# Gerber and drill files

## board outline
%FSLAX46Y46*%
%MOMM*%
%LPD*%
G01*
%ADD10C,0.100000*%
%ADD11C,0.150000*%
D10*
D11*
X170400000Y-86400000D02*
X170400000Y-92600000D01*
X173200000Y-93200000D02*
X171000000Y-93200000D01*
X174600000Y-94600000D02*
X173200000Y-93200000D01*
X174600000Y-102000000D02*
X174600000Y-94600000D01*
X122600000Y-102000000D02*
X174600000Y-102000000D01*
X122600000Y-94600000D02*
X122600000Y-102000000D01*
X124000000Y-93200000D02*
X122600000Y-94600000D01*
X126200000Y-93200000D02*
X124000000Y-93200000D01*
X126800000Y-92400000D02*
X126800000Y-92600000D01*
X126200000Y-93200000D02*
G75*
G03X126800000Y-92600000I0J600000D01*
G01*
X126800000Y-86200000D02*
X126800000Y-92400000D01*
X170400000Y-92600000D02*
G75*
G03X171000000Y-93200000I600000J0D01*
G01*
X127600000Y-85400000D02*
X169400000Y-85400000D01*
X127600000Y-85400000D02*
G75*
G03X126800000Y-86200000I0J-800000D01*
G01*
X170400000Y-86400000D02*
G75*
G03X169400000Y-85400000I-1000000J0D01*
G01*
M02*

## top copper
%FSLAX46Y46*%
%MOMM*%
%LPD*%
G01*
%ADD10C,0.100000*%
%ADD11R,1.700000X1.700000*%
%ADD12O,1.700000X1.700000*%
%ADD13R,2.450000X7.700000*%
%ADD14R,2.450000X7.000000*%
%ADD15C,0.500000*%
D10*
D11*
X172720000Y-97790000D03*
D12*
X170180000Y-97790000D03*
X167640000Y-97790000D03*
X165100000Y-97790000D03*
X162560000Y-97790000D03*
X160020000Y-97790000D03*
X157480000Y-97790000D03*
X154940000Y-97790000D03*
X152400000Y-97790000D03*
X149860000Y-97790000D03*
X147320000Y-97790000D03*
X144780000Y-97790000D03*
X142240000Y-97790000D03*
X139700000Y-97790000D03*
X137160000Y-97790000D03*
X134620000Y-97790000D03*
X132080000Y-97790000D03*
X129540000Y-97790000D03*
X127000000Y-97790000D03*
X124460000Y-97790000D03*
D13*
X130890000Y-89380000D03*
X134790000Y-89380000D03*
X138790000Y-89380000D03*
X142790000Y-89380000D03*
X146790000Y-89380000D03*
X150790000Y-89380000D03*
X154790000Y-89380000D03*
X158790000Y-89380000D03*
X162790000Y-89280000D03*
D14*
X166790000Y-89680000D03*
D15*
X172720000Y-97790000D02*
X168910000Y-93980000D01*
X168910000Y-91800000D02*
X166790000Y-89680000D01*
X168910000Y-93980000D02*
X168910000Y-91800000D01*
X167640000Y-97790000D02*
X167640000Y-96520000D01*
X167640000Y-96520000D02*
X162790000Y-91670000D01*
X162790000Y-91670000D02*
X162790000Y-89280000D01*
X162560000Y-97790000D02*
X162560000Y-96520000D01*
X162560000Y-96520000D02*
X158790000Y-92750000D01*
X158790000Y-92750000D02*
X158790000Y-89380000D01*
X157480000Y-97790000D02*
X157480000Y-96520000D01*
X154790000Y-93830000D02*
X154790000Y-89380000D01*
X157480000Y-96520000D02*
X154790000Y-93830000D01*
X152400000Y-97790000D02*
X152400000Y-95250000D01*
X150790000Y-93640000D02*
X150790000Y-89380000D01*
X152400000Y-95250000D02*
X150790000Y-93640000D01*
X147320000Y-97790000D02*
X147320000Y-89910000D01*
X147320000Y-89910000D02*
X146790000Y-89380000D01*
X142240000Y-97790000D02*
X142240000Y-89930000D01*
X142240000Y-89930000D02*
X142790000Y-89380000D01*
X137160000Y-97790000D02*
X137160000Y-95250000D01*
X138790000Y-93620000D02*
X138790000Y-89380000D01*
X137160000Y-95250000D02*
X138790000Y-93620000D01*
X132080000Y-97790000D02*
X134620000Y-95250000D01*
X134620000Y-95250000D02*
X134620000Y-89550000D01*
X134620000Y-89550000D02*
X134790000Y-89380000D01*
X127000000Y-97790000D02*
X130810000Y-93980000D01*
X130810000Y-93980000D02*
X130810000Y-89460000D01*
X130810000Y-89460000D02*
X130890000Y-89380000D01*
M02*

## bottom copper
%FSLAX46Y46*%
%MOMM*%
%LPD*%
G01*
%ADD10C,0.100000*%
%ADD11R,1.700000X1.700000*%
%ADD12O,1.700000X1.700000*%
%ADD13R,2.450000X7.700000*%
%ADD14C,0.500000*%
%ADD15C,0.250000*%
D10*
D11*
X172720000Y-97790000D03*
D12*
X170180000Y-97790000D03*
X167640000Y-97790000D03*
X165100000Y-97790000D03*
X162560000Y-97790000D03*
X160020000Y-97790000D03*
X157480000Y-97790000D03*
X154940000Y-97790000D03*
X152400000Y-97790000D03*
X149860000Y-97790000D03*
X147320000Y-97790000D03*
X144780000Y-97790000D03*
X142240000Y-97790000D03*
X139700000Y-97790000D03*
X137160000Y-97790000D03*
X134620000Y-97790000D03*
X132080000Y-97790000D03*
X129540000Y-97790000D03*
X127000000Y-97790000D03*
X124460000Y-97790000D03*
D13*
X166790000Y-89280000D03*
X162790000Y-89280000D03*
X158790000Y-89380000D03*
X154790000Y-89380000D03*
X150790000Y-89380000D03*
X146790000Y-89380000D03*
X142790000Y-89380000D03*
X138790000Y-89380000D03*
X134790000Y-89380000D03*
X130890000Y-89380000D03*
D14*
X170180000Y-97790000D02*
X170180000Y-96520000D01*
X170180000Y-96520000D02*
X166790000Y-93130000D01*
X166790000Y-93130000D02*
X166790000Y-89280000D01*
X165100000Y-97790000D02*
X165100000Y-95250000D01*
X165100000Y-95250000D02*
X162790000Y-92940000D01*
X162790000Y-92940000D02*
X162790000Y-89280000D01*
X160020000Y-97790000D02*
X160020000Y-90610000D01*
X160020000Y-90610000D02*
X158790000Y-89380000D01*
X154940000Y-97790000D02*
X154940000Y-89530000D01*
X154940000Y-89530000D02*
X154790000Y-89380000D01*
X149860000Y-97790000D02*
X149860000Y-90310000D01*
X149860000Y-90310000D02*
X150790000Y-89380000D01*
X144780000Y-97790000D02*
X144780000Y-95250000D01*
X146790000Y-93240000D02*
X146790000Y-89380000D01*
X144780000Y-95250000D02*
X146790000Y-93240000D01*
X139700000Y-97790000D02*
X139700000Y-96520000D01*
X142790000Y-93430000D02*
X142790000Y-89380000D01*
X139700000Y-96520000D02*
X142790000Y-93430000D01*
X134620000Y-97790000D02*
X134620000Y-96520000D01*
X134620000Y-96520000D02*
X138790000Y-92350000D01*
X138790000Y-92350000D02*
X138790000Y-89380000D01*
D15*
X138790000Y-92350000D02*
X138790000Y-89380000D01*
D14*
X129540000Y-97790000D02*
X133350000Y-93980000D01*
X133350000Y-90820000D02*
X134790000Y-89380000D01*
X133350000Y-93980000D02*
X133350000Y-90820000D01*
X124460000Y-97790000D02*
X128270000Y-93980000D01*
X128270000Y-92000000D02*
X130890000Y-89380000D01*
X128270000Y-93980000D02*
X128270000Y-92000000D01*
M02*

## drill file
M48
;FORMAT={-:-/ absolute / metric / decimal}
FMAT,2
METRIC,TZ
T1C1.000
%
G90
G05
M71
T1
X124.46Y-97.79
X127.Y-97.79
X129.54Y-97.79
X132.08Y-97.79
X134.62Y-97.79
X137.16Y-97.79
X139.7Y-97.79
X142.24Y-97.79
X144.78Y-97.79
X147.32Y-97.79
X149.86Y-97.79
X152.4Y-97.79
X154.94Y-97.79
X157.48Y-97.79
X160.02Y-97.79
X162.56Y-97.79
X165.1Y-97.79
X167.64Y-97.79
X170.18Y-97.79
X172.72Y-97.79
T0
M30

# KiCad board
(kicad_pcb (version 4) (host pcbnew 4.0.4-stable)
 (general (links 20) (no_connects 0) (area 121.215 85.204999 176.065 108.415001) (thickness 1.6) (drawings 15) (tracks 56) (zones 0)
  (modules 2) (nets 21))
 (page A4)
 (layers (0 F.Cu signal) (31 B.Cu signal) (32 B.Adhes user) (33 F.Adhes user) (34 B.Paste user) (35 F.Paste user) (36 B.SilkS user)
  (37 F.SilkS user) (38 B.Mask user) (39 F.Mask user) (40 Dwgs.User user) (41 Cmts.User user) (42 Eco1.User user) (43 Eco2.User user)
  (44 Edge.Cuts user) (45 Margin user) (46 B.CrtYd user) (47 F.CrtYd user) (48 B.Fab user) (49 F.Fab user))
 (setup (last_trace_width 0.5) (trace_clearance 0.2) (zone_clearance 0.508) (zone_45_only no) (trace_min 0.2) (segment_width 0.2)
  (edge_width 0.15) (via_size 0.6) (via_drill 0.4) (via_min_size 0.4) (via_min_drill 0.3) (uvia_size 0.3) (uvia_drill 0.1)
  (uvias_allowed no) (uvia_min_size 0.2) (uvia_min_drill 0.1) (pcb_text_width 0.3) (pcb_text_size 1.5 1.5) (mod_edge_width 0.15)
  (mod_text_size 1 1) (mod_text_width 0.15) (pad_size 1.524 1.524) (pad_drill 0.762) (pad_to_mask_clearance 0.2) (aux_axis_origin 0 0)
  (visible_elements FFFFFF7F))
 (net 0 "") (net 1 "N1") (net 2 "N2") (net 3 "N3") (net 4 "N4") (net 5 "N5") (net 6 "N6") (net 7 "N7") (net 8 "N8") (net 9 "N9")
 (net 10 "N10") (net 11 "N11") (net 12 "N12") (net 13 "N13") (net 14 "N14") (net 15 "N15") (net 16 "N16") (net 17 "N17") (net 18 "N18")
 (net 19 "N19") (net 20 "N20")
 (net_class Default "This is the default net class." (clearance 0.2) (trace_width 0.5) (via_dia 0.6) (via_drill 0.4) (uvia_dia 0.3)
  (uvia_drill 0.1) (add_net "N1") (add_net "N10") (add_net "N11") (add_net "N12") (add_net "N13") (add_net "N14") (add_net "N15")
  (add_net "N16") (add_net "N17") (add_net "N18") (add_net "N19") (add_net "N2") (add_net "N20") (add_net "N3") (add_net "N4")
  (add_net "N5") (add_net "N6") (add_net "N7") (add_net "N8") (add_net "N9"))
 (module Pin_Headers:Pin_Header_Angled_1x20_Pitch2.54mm (layer F.Cu) (at 172.72 97.79 270)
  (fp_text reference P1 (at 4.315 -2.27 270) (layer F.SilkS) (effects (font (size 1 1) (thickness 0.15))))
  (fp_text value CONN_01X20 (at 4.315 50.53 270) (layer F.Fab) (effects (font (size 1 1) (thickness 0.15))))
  (pad 1 thru_hole rect (at 0 0 270) (size 1.7 1.7) (drill 1) (layers *.Cu *.Mask) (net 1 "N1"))
  (pad 2 thru_hole oval (at 0 2.54 270) (size 1.7 1.7) (drill 1) (layers *.Cu *.Mask) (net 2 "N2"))
  (pad 3 thru_hole oval (at 0 5.08 270) (size 1.7 1.7) (drill 1) (layers *.Cu *.Mask) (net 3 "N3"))
  (pad 4 thru_hole oval (at 0 7.62 270) (size 1.7 1.7) (drill 1) (layers *.Cu *.Mask) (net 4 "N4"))
  (pad 5 thru_hole oval (at 0 10.16 270) (size 1.7 1.7) (drill 1) (layers *.Cu *.Mask) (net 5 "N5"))
  (pad 6 thru_hole oval (at 0 12.7 270) (size 1.7 1.7) (drill 1) (layers *.Cu *.Mask) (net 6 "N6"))
  (pad 7 thru_hole oval (at 0 15.24 270) (size 1.7 1.7) (drill 1) (layers *.Cu *.Mask) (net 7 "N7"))
  (pad 8 thru_hole oval (at 0 17.78 270) (size 1.7 1.7) (drill 1) (layers *.Cu *.Mask) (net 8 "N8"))
  (pad 9 thru_hole oval (at 0 20.32 270) (size 1.7 1.7) (drill 1) (layers *.Cu *.Mask) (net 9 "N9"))
  (pad 10 thru_hole oval (at 0 22.86 270) (size 1.7 1.7) (drill 1) (layers *.Cu *.Mask) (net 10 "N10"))
  (pad 11 thru_hole oval (at 0 25.4 270) (size 1.7 1.7) (drill 1) (layers *.Cu *.Mask) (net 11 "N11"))
  (pad 12 thru_hole oval (at 0 27.94 270) (size 1.7 1.7) (drill 1) (layers *.Cu *.Mask) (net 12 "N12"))
  (pad 13 thru_hole oval (at 0 30.48 270) (size 1.7 1.7) (drill 1) (layers *.Cu *.Mask) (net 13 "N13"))
  (pad 14 thru_hole oval (at 0 33.02 270) (size 1.7 1.7) (drill 1) (layers *.Cu *.Mask) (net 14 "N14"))
  (pad 15 thru_hole oval (at 0 35.56 270) (size 1.7 1.7) (drill 1) (layers *.Cu *.Mask) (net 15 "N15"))
  (pad 16 thru_hole oval (at 0 38.1 270) (size 1.7 1.7) (drill 1) (layers *.Cu *.Mask) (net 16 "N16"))
  (pad 17 thru_hole oval (at 0 40.64 270) (size 1.7 1.7) (drill 1) (layers *.Cu *.Mask) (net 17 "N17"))
  (pad 18 thru_hole oval (at 0 43.18 270) (size 1.7 1.7) (drill 1) (layers *.Cu *.Mask) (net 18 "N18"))
  (pad 19 thru_hole oval (at 0 45.72 270) (size 1.7 1.7) (drill 1) (layers *.Cu *.Mask) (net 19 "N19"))
  (pad 20 thru_hole oval (at 0 48.26 270) (size 1.7 1.7) (drill 1) (layers *.Cu *.Mask) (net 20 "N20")))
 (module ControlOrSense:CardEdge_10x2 (layer F.Cu) (at 148.59 93.98)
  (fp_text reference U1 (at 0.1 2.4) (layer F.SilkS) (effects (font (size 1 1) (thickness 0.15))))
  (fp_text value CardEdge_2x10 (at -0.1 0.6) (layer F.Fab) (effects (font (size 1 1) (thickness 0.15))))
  (pad A smd rect (at -17.7 -4.6) (size 2.45 7.7) (layers F.Cu F.Paste F.Mask) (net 19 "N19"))
  (pad B smd rect (at -13.8 -4.6) (size 2.45 7.7) (layers F.Cu F.Paste F.Mask) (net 17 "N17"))
  (pad C smd rect (at -9.8 -4.6) (size 2.45 7.7) (layers F.Cu F.Paste F.Mask) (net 15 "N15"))
  (pad D smd rect (at -5.8 -4.6) (size 2.45 7.7) (layers F.Cu F.Paste F.Mask) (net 13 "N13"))
  (pad E smd rect (at -1.8 -4.6) (size 2.45 7.7) (layers F.Cu F.Paste F.Mask) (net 11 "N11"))
  (pad F smd rect (at 2.2 -4.6) (size 2.45 7.7) (layers F.Cu F.Paste F.Mask) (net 9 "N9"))
  (pad G smd rect (at 6.2 -4.6) (size 2.45 7.7) (layers F.Cu F.Paste F.Mask) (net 7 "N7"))
  (pad H smd rect (at 10.2 -4.6) (size 2.45 7.7) (layers F.Cu F.Paste F.Mask) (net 5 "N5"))
  (pad I smd rect (at 14.2 -4.7) (size 2.45 7.7) (layers F.Cu F.Paste F.Mask) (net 3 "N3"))
  (pad J smd rect (at 18.2 -4.3) (size 2.45 7) (layers F.Cu F.Paste F.Mask) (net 1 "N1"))
  (pad 10 smd rect (at 18.2 -4.7) (size 2.45 7.7) (layers B.Cu F.Paste F.Mask) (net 2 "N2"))
  (pad 9 smd rect (at 14.2 -4.7) (size 2.45 7.7) (layers B.Cu F.Paste F.Mask) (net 4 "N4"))
  (pad 8 smd rect (at 10.2 -4.6) (size 2.45 7.7) (layers B.Cu F.Paste F.Mask) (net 6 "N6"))
  (pad 7 smd rect (at 6.2 -4.6) (size 2.45 7.7) (layers B.Cu F.Paste F.Mask) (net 8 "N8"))
  (pad 6 smd rect (at 2.2 -4.6) (size 2.45 7.7) (layers B.Cu F.Paste F.Mask) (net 10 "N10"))
  (pad 5 smd rect (at -1.8 -4.6) (size 2.45 7.7) (layers B.Cu F.Paste F.Mask) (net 12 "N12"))
  (pad 4 smd rect (at -5.8 -4.6) (size 2.45 7.7) (layers B.Cu F.Paste F.Mask) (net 14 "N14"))
  (pad 3 smd rect (at -9.8 -4.6) (size 2.45 7.7) (layers B.Cu F.Paste F.Mask) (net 16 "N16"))
  (pad 2 smd rect (at -13.8 -4.6) (size 2.45 7.7) (layers B.Cu F.Paste B.Mask) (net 18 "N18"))
  (pad 1 smd rect (at -17.7 -4.6) (size 2.45 7.7) (layers B.Cu F.Paste B.Mask) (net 20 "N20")))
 (gr_line (start 170.4 86.4) (end 170.4 92.6) (angle 90) (layer Edge.Cuts) (width 0.15))
 (gr_line (start 173.2 93.2) (end 171 93.2) (angle 90) (layer Edge.Cuts) (width 0.15))
 (gr_line (start 174.6 94.6) (end 173.2 93.2) (angle 90) (layer Edge.Cuts) (width 0.15))
 (gr_line (start 174.6 102) (end 174.6 94.6) (angle 90) (layer Edge.Cuts) (width 0.15))
 (gr_line (start 122.6 102) (end 174.6 102) (angle 90) (layer Edge.Cuts) (width 0.15))
 (gr_line (start 122.6 94.6) (end 122.6 102) (angle 90) (layer Edge.Cuts) (width 0.15))
 (gr_line (start 124 93.2) (end 122.6 94.6) (angle 90) (layer Edge.Cuts) (width 0.15))
 (gr_line (start 126.2 93.2) (end 124 93.2) (angle 90) (layer Edge.Cuts) (width 0.15))
 (gr_line (start 126.8 92.4) (end 126.8 92.6) (angle 90) (layer Edge.Cuts) (width 0.15))
 (gr_arc (start 126.2 92.6) (end 126.8 92.6) (angle 90) (layer Edge.Cuts) (width 0.15))
 (gr_line (start 126.8 86.2) (end 126.8 92.4) (angle 90) (layer Edge.Cuts) (width 0.15))
 (gr_arc (start 171 92.6) (end 171 93.2) (angle 90) (layer Edge.Cuts) (width 0.15))
 (gr_line (start 127.6 85.4) (end 169.4 85.4) (angle 90) (layer Edge.Cuts) (width 0.15))
 (gr_arc (start 127.6 86.2) (end 126.8 86.2) (angle 90) (layer Edge.Cuts) (width 0.15))
 (gr_arc (start 169.4 86.4) (end 169.4 85.4) (angle 90) (layer Edge.Cuts) (width 0.15))
 (segment (start 172.72 97.79) (end 168.91 93.98) (width 0.5) (layer F.Cu) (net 1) (status 400000))
 (segment (start 168.91 91.8) (end 166.79 89.68) (width 0.5) (layer F.Cu) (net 1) (status 800000))
 (segment (start 168.91 93.98) (end 168.91 91.8) (width 0.5) (layer F.Cu) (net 1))
 (segment (start 170.18 97.79) (end 170.18 96.52) (width 0.5) (layer B.Cu) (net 2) (status 400000))
 (segment (start 170.18 96.52) (end 166.79 93.13) (width 0.5) (layer B.Cu) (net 2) (status 800000))
 (segment (start 166.79 93.13) (end 166.79 89.28) (width 0.5) (layer B.Cu) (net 2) (status C00000))
 (segment (start 167.64 97.79) (end 167.64 96.52) (width 0.5) (layer F.Cu) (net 3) (status 400000))
 (segment (start 167.64 96.52) (end 162.79 91.67) (width 0.5) (layer F.Cu) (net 3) (status 800000))
 (segment (start 162.79 91.67) (end 162.79 89.28) (width 0.5) (layer F.Cu) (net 3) (status C00000))
 (segment (start 165.1 97.79) (end 165.1 95.25) (width 0.5) (layer B.Cu) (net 4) (status 400000))
 (segment (start 165.1 95.25) (end 162.79 92.94) (width 0.5) (layer B.Cu) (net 4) (status 800000))
 (segment (start 162.79 92.94) (end 162.79 89.28) (width 0.5) (layer B.Cu) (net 4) (status C00000))
 (segment (start 162.56 97.79) (end 162.56 96.52) (width 0.5) (layer F.Cu) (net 5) (status 400000))
 (segment (start 162.56 96.52) (end 158.79 92.75) (width 0.5) (layer F.Cu) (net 5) (status 800000))
 (segment (start 158.79 92.75) (end 158.79 89.38) (width 0.5) (layer F.Cu) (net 5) (status C00000))
 (segment (start 160.02 97.79) (end 160.02 90.61) (width 0.5) (layer B.Cu) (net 6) (status 400000))
 (segment (start 160.02 90.61) (end 158.79 89.38) (width 0.5) (layer B.Cu) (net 6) (status 800000))
 (segment (start 157.48 97.79) (end 157.48 96.52) (width 0.5) (layer F.Cu) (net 7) (status 400000))
 (segment (start 154.79 93.83) (end 154.79 89.38) (width 0.5) (layer F.Cu) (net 7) (status 800000))
 (segment (start 157.48 96.52) (end 154.79 93.83) (width 0.5) (layer F.Cu) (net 7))
 (segment (start 154.94 97.79) (end 154.94 89.53) (width 0.5) (layer B.Cu) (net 8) (status C00000))
 (segment (start 154.94 89.53) (end 154.79 89.38) (width 0.5) (layer B.Cu) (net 8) (status C00000))
 (segment (start 152.4 97.79) (end 152.4 95.25) (width 0.5) (layer F.Cu) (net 9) (status 400000))
 (segment (start 150.79 93.64) (end 150.79 89.38) (width 0.5) (layer F.Cu) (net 9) (status 800000))
 (segment (start 152.4 95.25) (end 150.79 93.64) (width 0.5) (layer F.Cu) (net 9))
 (segment (start 149.86 97.79) (end 149.86 90.31) (width 0.5) (layer B.Cu) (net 10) (status C00000))
 (segment (start 149.86 90.31) (end 150.79 89.38) (width 0.5) (layer B.Cu) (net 10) (status C00000))
 (segment (start 147.32 97.79) (end 147.32 89.91) (width 0.5) (layer F.Cu) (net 11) (status C00000))
 (segment (start 147.32 89.91) (end 146.79 89.38) (width 0.5) (layer F.Cu) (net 11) (status C00000))
 (segment (start 144.78 97.79) (end 144.78 95.25) (width 0.5) (layer B.Cu) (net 12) (status 400000))
 (segment (start 146.79 93.24) (end 146.79 89.38) (width 0.5) (layer B.Cu) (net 12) (status 800000))
 (segment (start 144.78 95.25) (end 146.79 93.24) (width 0.5) (layer B.Cu) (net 12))
 (segment (start 142.24 97.79) (end 142.24 89.93) (width 0.5) (layer F.Cu) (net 13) (status C00000))
 (segment (start 142.24 89.93) (end 142.79 89.38) (width 0.5) (layer F.Cu) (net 13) (status C00000))
 (segment (start 139.7 97.79) (end 139.7 96.52) (width 0.5) (layer B.Cu) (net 14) (status 400000))
 (segment (start 142.79 93.43) (end 142.79 89.38) (width 0.5) (layer B.Cu) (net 14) (status 800000))
 (segment (start 139.7 96.52) (end 142.79 93.43) (width 0.5) (layer B.Cu) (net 14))
 (segment (start 137.16 97.79) (end 137.16 95.25) (width 0.5) (layer F.Cu) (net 15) (status 400000))
 (segment (start 138.79 93.62) (end 138.79 89.38) (width 0.5) (layer F.Cu) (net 15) (status 800000))
 (segment (start 137.16 95.25) (end 138.79 93.62) (width 0.5) (layer F.Cu) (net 15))
 (segment (start 134.62 97.79) (end 134.62 96.52) (width 0.5) (layer B.Cu) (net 16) (status 400000))
 (segment (start 134.62 96.52) (end 138.79 92.35) (width 0.5) (layer B.Cu) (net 16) (status 800000))
 (segment (start 138.79 92.35) (end 138.79 89.38) (width 0.5) (layer B.Cu) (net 16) (status C00000))
 (segment (start 138.79 92.35) (end 138.79 89.38) (width 0.25) (layer B.Cu) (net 16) (status C00000))
 (segment (start 132.08 97.79) (end 134.62 95.25) (width 0.5) (layer F.Cu) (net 17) (status 400000))
 (segment (start 134.62 95.25) (end 134.62 89.55) (width 0.5) (layer F.Cu) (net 17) (status 800000))
 (segment (start 134.62 89.55) (end 134.79 89.38) (width 0.5) (layer F.Cu) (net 17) (status C00000))
 (segment (start 129.54 97.79) (end 133.35 93.98) (width 0.5) (layer B.Cu) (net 18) (status 400000))
 (segment (start 133.35 90.82) (end 134.79 89.38) (width 0.5) (layer B.Cu) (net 18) (status 800000))
 (segment (start 133.35 93.98) (end 133.35 90.82) (width 0.5) (layer B.Cu) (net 18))
 (segment (start 127 97.79) (end 130.81 93.98) (width 0.5) (layer F.Cu) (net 19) (status 400000))
 (segment (start 130.81 93.98) (end 130.81 89.46) (width 0.5) (layer F.Cu) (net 19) (status 800000))
 (segment (start 130.81 89.46) (end 130.89 89.38) (width 0.5) (layer F.Cu) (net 19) (status C00000))
 (segment (start 124.46 97.79) (end 128.27 93.98) (width 0.5) (layer B.Cu) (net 20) (status 400000))
 (segment (start 128.27 92) (end 130.89 89.38) (width 0.5) (layer B.Cu) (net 20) (status 800000))
 (segment (start 128.27 93.98) (end 128.27 92) (width 0.5) (layer B.Cu) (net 20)))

